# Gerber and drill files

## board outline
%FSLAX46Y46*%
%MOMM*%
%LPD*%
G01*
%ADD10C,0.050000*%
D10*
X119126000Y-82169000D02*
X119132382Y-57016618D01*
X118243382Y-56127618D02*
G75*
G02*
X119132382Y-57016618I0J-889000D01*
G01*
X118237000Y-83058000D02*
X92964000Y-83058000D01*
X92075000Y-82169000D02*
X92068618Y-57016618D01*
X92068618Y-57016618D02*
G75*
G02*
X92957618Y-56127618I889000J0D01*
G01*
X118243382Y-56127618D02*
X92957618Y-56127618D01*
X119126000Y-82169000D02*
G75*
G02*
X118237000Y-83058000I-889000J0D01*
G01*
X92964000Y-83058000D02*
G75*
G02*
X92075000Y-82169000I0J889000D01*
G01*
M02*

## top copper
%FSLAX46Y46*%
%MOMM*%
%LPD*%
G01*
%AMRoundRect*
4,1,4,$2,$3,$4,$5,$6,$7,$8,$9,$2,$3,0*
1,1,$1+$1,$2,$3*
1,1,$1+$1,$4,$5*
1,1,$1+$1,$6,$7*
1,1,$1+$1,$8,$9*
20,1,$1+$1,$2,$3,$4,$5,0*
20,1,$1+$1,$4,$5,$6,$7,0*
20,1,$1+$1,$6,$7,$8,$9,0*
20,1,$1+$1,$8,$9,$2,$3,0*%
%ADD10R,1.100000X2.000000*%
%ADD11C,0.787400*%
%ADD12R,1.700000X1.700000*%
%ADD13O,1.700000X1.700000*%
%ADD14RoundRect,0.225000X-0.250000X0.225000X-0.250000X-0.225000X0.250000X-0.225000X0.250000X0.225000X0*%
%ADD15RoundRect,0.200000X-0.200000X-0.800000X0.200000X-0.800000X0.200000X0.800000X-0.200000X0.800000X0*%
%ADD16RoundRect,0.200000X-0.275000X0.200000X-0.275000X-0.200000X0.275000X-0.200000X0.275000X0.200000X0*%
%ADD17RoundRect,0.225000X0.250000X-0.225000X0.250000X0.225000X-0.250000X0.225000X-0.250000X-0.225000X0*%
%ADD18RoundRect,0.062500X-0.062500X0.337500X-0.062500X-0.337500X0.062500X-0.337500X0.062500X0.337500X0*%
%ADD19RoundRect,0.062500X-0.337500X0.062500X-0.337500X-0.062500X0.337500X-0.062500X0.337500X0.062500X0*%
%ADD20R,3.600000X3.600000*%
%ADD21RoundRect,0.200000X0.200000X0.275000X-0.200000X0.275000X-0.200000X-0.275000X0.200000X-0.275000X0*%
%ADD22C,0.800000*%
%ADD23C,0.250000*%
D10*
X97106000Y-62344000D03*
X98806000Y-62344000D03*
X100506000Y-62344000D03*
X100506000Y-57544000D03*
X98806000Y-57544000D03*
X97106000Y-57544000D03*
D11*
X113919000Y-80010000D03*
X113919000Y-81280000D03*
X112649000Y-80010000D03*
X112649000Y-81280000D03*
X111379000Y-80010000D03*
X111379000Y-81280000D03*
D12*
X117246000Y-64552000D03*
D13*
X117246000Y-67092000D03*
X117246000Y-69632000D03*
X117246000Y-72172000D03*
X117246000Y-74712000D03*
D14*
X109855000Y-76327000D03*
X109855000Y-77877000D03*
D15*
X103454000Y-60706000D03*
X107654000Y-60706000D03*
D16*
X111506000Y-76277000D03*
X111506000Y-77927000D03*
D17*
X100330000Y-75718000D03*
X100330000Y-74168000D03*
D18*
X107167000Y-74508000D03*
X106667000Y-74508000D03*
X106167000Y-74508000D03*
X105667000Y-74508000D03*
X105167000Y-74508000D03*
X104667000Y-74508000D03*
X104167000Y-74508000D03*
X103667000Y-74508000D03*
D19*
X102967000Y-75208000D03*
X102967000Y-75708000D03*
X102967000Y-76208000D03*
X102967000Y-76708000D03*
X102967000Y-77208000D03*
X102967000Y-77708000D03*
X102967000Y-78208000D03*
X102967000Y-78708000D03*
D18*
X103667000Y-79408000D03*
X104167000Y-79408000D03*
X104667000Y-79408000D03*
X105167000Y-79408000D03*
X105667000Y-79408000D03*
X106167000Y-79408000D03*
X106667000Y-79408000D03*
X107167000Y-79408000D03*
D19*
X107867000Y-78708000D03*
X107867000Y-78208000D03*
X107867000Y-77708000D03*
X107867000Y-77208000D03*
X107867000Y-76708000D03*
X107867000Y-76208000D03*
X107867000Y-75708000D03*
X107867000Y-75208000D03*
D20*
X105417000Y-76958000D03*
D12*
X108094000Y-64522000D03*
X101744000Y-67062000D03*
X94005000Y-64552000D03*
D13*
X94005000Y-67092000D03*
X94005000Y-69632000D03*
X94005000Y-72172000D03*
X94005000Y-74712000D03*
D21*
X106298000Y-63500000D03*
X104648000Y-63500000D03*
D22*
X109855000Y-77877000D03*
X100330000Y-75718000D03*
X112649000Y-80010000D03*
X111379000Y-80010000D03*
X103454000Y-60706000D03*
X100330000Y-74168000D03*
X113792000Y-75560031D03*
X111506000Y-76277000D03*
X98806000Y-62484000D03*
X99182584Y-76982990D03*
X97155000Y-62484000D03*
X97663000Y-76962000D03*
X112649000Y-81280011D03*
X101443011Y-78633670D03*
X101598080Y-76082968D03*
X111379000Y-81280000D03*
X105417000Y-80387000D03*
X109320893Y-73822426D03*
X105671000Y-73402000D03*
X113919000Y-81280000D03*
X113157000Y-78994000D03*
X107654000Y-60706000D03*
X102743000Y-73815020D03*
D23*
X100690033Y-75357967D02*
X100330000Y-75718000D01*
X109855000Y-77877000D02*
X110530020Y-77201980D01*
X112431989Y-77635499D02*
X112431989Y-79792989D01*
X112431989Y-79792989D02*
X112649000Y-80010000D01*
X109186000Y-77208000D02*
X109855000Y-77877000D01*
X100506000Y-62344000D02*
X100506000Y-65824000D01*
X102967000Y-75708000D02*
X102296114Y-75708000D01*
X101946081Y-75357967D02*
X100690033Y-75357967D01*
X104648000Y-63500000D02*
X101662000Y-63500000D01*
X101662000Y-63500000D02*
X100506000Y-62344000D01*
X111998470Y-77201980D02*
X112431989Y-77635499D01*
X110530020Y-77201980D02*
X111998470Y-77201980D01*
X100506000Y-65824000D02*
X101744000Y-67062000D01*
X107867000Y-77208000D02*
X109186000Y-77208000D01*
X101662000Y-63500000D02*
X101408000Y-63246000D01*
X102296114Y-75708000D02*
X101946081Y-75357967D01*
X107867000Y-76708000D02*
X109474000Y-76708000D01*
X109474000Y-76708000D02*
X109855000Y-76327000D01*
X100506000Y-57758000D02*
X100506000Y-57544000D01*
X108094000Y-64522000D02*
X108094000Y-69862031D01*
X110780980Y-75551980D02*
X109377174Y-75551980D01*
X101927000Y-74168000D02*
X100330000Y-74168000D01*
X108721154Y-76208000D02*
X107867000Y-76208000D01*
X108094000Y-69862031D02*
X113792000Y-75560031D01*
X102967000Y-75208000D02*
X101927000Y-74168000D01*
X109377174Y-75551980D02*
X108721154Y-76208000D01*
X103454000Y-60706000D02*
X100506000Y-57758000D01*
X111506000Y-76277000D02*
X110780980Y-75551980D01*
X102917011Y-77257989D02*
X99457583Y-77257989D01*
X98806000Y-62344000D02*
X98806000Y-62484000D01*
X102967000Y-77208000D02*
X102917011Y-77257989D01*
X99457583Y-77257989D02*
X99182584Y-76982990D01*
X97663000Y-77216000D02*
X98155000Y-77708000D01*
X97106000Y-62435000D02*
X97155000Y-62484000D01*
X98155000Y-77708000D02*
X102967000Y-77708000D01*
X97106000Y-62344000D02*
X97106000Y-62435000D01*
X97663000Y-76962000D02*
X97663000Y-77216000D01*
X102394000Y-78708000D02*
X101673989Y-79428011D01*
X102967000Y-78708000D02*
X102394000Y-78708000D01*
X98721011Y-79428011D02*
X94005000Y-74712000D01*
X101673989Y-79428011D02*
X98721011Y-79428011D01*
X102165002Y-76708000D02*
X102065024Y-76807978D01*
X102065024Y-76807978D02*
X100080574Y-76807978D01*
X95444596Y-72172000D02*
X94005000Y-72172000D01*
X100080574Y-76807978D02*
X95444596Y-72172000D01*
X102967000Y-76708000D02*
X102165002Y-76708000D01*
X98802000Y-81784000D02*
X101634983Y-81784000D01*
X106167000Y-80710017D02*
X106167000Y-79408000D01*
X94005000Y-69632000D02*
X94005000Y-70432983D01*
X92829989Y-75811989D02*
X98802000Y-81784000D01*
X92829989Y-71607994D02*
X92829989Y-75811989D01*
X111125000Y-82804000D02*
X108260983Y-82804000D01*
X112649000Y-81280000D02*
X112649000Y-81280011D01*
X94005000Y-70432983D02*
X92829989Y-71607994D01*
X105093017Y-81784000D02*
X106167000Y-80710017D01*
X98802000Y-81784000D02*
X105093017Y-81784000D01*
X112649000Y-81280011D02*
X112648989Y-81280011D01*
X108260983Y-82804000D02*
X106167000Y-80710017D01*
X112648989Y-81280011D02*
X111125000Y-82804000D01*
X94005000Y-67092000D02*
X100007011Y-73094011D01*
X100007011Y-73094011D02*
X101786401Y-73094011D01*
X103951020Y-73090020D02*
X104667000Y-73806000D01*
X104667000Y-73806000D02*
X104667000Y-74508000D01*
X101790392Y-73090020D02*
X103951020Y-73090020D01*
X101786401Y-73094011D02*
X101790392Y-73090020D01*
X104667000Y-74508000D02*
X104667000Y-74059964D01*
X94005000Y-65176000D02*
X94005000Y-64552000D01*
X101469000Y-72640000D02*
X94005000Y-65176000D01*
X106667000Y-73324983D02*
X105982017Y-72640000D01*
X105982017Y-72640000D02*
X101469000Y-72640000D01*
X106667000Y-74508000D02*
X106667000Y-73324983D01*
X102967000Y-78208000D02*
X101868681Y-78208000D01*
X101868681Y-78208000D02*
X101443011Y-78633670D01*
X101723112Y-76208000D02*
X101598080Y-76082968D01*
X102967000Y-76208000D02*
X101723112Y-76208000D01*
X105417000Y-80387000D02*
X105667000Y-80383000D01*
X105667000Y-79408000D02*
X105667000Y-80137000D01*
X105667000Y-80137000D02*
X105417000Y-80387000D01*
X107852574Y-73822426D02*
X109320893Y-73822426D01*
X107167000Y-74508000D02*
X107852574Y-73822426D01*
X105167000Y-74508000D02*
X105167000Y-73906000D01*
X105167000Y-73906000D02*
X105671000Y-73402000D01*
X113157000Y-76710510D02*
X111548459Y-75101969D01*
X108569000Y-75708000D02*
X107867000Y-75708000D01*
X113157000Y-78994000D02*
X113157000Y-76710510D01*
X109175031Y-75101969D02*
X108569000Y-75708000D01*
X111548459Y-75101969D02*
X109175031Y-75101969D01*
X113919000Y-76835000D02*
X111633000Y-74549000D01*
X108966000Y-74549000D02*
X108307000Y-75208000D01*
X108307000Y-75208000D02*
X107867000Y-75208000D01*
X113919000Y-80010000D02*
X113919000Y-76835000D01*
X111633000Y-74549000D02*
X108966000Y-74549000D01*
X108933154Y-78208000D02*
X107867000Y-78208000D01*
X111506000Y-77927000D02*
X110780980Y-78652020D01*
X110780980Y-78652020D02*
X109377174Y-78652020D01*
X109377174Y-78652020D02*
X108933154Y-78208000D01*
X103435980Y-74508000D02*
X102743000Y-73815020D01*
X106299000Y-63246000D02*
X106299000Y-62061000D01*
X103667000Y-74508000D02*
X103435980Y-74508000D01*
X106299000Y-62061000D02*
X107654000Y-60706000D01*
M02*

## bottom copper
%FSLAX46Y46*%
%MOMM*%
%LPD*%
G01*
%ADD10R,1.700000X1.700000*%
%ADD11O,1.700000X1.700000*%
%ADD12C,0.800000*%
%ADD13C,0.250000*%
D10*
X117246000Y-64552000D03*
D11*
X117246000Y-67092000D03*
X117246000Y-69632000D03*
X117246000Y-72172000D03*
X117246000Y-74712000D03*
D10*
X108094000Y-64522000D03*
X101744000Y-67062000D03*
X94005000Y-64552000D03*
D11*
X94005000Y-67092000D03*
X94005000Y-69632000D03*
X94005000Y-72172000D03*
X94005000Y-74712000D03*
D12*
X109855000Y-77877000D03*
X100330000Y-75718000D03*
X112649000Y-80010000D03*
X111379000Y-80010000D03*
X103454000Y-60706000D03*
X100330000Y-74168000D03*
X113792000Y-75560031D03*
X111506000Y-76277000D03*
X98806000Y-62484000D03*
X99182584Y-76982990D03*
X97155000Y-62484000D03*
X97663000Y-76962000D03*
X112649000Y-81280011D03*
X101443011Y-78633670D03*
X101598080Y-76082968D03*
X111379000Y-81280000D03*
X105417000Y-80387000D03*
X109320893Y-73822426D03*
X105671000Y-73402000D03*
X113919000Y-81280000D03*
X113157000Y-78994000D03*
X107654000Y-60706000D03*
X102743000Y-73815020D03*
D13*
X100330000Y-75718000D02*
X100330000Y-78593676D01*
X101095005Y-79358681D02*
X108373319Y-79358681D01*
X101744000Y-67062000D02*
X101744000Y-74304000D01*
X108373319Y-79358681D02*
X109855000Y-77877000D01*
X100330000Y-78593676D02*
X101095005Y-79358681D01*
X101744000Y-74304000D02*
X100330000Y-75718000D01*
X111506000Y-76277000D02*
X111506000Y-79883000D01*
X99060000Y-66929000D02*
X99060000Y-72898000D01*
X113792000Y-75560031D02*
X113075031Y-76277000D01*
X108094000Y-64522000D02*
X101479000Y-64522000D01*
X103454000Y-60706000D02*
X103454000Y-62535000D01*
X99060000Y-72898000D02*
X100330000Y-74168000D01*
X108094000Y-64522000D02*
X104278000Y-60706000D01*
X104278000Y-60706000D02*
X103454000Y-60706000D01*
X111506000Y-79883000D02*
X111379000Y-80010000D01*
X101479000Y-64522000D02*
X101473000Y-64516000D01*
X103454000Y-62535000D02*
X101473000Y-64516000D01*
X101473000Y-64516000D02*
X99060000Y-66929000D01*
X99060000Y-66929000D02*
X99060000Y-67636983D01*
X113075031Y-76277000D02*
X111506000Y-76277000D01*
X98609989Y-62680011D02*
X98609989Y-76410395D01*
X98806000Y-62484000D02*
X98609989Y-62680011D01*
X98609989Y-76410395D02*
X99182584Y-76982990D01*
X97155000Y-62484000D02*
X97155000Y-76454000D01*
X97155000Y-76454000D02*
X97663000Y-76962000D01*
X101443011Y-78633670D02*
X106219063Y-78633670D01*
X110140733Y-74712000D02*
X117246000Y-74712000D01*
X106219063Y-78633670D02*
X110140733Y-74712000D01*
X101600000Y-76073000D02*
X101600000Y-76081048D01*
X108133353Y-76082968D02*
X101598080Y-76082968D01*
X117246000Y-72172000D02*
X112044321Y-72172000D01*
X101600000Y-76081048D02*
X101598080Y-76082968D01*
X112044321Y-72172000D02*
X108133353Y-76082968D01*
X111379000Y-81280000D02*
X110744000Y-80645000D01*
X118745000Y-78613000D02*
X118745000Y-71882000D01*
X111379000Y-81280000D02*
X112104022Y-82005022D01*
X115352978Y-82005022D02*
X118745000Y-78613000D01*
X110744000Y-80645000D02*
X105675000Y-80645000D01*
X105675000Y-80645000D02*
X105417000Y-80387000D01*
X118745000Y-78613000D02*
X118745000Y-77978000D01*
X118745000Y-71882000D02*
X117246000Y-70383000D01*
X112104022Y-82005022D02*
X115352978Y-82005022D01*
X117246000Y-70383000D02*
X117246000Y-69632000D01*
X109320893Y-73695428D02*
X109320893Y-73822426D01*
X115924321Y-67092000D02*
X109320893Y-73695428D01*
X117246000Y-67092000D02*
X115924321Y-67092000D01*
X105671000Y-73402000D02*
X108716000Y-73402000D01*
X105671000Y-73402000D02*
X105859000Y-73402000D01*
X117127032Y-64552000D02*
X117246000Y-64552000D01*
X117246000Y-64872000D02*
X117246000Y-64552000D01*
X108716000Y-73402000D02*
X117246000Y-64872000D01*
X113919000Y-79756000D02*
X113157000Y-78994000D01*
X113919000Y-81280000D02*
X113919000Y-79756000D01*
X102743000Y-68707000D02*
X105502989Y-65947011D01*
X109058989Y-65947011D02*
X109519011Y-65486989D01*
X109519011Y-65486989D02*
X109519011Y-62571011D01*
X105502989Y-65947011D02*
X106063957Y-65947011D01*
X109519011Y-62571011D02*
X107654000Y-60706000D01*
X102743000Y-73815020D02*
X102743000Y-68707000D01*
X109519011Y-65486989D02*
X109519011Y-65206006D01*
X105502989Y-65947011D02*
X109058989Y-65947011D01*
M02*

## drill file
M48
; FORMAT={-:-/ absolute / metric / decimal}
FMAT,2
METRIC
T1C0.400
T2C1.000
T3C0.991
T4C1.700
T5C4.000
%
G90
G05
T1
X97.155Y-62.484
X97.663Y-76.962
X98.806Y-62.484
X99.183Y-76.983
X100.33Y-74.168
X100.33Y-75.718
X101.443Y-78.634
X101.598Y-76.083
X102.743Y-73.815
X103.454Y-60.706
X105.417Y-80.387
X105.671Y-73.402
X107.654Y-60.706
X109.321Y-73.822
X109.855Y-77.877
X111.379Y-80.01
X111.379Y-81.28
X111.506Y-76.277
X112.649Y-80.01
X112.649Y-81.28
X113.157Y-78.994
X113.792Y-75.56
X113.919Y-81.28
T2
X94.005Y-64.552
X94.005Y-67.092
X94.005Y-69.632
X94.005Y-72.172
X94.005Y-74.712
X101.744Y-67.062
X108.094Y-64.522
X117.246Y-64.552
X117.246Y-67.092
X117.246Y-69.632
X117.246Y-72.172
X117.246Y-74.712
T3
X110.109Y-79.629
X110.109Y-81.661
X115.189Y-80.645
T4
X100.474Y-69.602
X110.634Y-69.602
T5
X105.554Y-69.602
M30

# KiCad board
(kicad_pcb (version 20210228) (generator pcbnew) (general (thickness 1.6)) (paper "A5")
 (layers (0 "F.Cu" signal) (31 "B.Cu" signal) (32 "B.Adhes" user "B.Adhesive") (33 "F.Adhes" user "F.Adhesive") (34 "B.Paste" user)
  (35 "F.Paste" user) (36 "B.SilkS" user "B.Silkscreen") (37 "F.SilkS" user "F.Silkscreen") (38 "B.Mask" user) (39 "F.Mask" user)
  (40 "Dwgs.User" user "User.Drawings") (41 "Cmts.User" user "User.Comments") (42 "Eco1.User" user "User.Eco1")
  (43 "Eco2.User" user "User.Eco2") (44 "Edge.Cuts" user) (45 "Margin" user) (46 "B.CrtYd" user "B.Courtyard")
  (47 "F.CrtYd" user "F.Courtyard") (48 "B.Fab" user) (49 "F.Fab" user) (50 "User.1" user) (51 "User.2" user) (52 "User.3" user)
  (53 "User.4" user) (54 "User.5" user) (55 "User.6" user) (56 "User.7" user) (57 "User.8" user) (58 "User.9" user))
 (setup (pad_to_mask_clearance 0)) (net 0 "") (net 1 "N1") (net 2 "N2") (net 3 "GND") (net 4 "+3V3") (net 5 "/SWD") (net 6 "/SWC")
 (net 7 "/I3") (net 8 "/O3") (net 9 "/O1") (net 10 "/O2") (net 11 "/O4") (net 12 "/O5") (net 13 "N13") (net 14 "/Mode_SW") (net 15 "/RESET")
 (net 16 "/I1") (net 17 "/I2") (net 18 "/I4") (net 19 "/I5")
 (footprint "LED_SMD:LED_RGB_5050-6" (layer "F.Cu") (at 98.806 59.944 90)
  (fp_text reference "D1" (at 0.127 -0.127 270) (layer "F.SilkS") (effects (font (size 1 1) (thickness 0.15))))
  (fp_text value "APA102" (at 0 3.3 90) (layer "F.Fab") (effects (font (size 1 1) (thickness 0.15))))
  (pad "1" smd rect (at -2.4 -1.7 180) (locked) (size 1.1 2) (layers "F.Cu" "F.Paste" "F.Mask") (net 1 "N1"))
  (pad "2" smd rect (at -2.4 0 180) (locked) (size 1.1 2) (layers "F.Cu" "F.Paste" "F.Mask") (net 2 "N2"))
  (pad "3" smd rect (at -2.4 1.7 180) (locked) (size 1.1 2) (layers "F.Cu" "F.Paste" "F.Mask") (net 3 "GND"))
  (pad "4" smd rect (at 2.4 1.7 180) (locked) (size 1.1 2) (layers "F.Cu" "F.Paste" "F.Mask") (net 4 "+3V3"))
  (pad "5" smd rect (at 2.4 0 180) (locked) (size 1.1 2) (layers "F.Cu" "F.Paste" "F.Mask"))
  (pad "6" smd rect (at 2.4 -1.7 180) (locked) (size 1.1 2) (layers "F.Cu" "F.Paste" "F.Mask")))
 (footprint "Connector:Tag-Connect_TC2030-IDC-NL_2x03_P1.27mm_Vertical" (layer "F.Cu") (at 112.649 80.645 180)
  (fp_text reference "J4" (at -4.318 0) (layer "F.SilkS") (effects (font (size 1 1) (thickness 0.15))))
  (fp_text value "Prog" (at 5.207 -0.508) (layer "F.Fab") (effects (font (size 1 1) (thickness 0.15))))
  (pad "" np_thru_hole circle (at 2.54 1.016 180) (locked) (size 0.9906 0.9906) (drill 0.9906) (layers *.Cu *.Mask))
  (pad "" np_thru_hole circle (at -2.54 0 180) (locked) (size 0.9906 0.9906) (drill 0.9906) (layers *.Cu *.Mask))
  (pad "" np_thru_hole circle (at 2.54 -1.016 180) (locked) (size 0.9906 0.9906) (drill 0.9906) (layers *.Cu *.Mask))
  (pad "1" connect circle (at -1.27 0.635 180) (locked) (size 0.7874 0.7874) (layers "F.Cu" "F.Mask") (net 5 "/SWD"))
  (pad "2" connect circle (at -1.27 -0.635 180) (locked) (size 0.7874 0.7874) (layers "F.Cu" "F.Mask") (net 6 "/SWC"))
  (pad "3" connect circle (at 0 0.635 180) (locked) (size 0.7874 0.7874) (layers "F.Cu" "F.Mask") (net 3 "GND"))
  (pad "4" connect circle (at 0 -0.635 180) (locked) (size 0.7874 0.7874) (layers "F.Cu" "F.Mask") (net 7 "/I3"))
  (pad "5" connect circle (at 1.27 0.635 180) (locked) (size 0.7874 0.7874) (layers "F.Cu" "F.Mask") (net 4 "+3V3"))
  (pad "6" connect circle (at 1.27 -0.635 180) (locked) (size 0.7874 0.7874) (layers "F.Cu" "F.Mask") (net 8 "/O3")))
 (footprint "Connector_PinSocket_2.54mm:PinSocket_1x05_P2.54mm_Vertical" (layer "F.Cu") (at 117.246 64.552)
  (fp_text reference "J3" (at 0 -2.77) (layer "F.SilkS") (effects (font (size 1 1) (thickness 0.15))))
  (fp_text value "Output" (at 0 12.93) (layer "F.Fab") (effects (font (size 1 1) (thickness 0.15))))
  (pad "1" thru_hole rect (at 0 0) (locked) (size 1.7 1.7) (drill 1) (layers *.Cu *.Mask) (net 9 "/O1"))
  (pad "2" thru_hole oval (at 0 2.54) (locked) (size 1.7 1.7) (drill 1) (layers *.Cu *.Mask) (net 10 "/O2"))
  (pad "3" thru_hole oval (at 0 5.08) (locked) (size 1.7 1.7) (drill 1) (layers *.Cu *.Mask) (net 8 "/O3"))
  (pad "4" thru_hole oval (at 0 7.62) (locked) (size 1.7 1.7) (drill 1) (layers *.Cu *.Mask) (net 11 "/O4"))
  (pad "5" thru_hole oval (at 0 10.16) (locked) (size 1.7 1.7) (drill 1) (layers *.Cu *.Mask) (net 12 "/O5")))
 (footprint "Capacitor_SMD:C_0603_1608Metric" (layer "F.Cu") (at 109.855 77.102 -90)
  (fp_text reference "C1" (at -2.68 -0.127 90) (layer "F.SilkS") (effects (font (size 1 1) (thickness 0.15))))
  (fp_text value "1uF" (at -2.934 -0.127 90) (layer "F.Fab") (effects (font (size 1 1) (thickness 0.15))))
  (pad "1" smd roundrect (at -0.775 0 270) (locked) (size 0.9 0.95) (layers "F.Cu" "F.Paste" "F.Mask") (roundrect_rratio 0.25)
   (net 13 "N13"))
  (pad "2" smd roundrect (at 0.775 0 270) (locked) (size 0.9 0.95) (layers "F.Cu" "F.Paste" "F.Mask") (roundrect_rratio 0.25) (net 3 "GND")))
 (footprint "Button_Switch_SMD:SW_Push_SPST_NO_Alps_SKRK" (layer "F.Cu") (at 105.554 60.706)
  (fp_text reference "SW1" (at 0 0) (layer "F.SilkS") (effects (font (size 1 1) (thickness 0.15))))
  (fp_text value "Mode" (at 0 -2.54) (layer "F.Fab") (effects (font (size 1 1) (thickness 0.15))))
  (pad "1" smd roundrect (at -2.1 0) (locked) (size 0.8 2) (layers "F.Cu" "F.Paste" "F.Mask") (roundrect_rratio 0.25) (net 4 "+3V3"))
  (pad "2" smd roundrect (at 2.1 0) (locked) (size 0.8 2) (layers "F.Cu" "F.Paste" "F.Mask") (roundrect_rratio 0.25) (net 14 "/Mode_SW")))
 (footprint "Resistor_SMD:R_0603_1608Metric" (layer "F.Cu") (at 111.506 77.102 -90)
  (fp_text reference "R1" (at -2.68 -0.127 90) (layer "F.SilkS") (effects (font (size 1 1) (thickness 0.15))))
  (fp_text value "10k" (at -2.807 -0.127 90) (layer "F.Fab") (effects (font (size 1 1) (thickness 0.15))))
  (pad "1" smd roundrect (at -0.825 0 270) (locked) (size 0.8 0.95) (layers "F.Cu" "F.Paste" "F.Mask") (roundrect_rratio 0.25)
   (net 4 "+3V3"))
  (pad "2" smd roundrect (at 0.825 0 270) (locked) (size 0.8 0.95) (layers "F.Cu" "F.Paste" "F.Mask") (roundrect_rratio 0.25)
   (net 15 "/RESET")))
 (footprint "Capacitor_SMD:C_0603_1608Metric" (layer "F.Cu") (at 100.33 74.943 90)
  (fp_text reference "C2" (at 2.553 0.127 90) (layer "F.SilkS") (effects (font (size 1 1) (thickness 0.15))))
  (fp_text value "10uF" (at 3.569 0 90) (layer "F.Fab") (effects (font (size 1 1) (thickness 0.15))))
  (pad "1" smd roundrect (at -0.775 0 90) (locked) (size 0.9 0.95) (layers "F.Cu" "F.Paste" "F.Mask") (roundrect_rratio 0.25) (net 3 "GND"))
  (pad "2" smd roundrect (at 0.775 0 90) (locked) (size 0.9 0.95) (layers "F.Cu" "F.Paste" "F.Mask") (roundrect_rratio 0.25) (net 4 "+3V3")))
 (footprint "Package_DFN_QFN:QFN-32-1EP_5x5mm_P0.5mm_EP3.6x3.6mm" (layer "F.Cu") (at 105.417 76.958 -90)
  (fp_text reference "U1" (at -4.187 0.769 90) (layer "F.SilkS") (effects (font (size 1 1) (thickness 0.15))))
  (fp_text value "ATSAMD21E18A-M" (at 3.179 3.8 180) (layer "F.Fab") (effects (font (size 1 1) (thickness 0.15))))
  (pad "" smd roundrect (at -1.2 1.2 270) (locked) (size 0.97 0.97) (layers "F.Paste") (roundrect_rratio 0.25))
  (pad "" smd roundrect (at 0 0 270) (locked) (size 0.97 0.97) (layers "F.Paste") (roundrect_rratio 0.25))
  (pad "" smd roundrect (at 1.2 -1.2 270) (locked) (size 0.97 0.97) (layers "F.Paste") (roundrect_rratio 0.25))
  (pad "" smd roundrect (at -1.2 -1.2 270) (locked) (size 0.97 0.97) (layers "F.Paste") (roundrect_rratio 0.25))
  (pad "" smd roundrect (at 0 1.2 270) (locked) (size 0.97 0.97) (layers "F.Paste") (roundrect_rratio 0.25))
  (pad "" smd roundrect (at 1.2 0 270) (locked) (size 0.97 0.97) (layers "F.Paste") (roundrect_rratio 0.25))
  (pad "" smd roundrect (at -1.2 0 270) (locked) (size 0.97 0.97) (layers "F.Paste") (roundrect_rratio 0.25))
  (pad "" smd roundrect (at 0 -1.2 270) (locked) (size 0.97 0.97) (layers "F.Paste") (roundrect_rratio 0.25))
  (pad "" smd roundrect (at 1.2 1.2 270) (locked) (size 0.97 0.97) (layers "F.Paste") (roundrect_rratio 0.25))
  (pad "1" smd roundrect (at -2.45 -1.75 270) (locked) (size 0.8 0.25) (layers "F.Cu" "F.Paste" "F.Mask") (roundrect_rratio 0.25)
   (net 10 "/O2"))
  (pad "2" smd roundrect (at -2.45 -1.25 270) (locked) (size 0.8 0.25) (layers "F.Cu" "F.Paste" "F.Mask") (roundrect_rratio 0.25)
   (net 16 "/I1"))
  (pad "3" smd roundrect (at -2.45 -0.75 270) (locked) (size 0.8 0.25) (layers "F.Cu" "F.Paste" "F.Mask") (roundrect_rratio 0.25))
  (pad "4" smd roundrect (at -2.45 -0.25 270) (locked) (size 0.8 0.25) (layers "F.Cu" "F.Paste" "F.Mask") (roundrect_rratio 0.25))
  (pad "5" smd roundrect (at -2.45 0.25 270) (locked) (size 0.8 0.25) (layers "F.Cu" "F.Paste" "F.Mask") (roundrect_rratio 0.25)
   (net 9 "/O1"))
  (pad "6" smd roundrect (at -2.45 0.75 270) (locked) (size 0.8 0.25) (layers "F.Cu" "F.Paste" "F.Mask") (roundrect_rratio 0.25)
   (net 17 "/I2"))
  (pad "7" smd roundrect (at -2.45 1.25 270) (locked) (size 0.8 0.25) (layers "F.Cu" "F.Paste" "F.Mask") (roundrect_rratio 0.25))
  (pad "8" smd roundrect (at -2.45 1.75 270) (locked) (size 0.8 0.25) (layers "F.Cu" "F.Paste" "F.Mask") (roundrect_rratio 0.25)
   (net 14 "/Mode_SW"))
  (pad "9" smd roundrect (at -1.75 2.45 270) (locked) (size 0.25 0.8) (layers "F.Cu" "F.Paste" "F.Mask") (roundrect_rratio 0.25)
   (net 4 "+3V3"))
  (pad "10" smd roundrect (at -1.25 2.45 270) (locked) (size 0.25 0.8) (layers "F.Cu" "F.Paste" "F.Mask") (roundrect_rratio 0.25)
   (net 3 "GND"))
  (pad "11" smd roundrect (at -0.75 2.45 270) (locked) (size 0.25 0.8) (layers "F.Cu" "F.Paste" "F.Mask") (roundrect_rratio 0.25)
   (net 11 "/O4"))
  (pad "12" smd roundrect (at -0.25 2.45 270) (locked) (size 0.25 0.8) (layers "F.Cu" "F.Paste" "F.Mask") (roundrect_rratio 0.25)
   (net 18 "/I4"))
  (pad "13" smd roundrect (at 0.25 2.45 270) (locked) (size 0.25 0.8) (layers "F.Cu" "F.Paste" "F.Mask") (roundrect_rratio 0.25)
   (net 2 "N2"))
  (pad "14" smd roundrect (at 0.75 2.45 270) (locked) (size 0.25 0.8) (layers "F.Cu" "F.Paste" "F.Mask") (roundrect_rratio 0.25)
   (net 1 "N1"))
  (pad "15" smd roundrect (at 1.25 2.45 270) (locked) (size 0.25 0.8) (layers "F.Cu" "F.Paste" "F.Mask") (roundrect_rratio 0.25)
   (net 12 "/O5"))
  (pad "16" smd roundrect (at 1.75 2.45 270) (locked) (size 0.25 0.8) (layers "F.Cu" "F.Paste" "F.Mask") (roundrect_rratio 0.25)
   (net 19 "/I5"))
  (pad "17" smd roundrect (at 2.45 1.75 270) (locked) (size 0.8 0.25) (layers "F.Cu" "F.Paste" "F.Mask") (roundrect_rratio 0.25))
  (pad "18" smd roundrect (at 2.45 1.25 270) (locked) (size 0.8 0.25) (layers "F.Cu" "F.Paste" "F.Mask") (roundrect_rratio 0.25))
  (pad "19" smd roundrect (at 2.45 0.75 270) (locked) (size 0.8 0.25) (layers "F.Cu" "F.Paste" "F.Mask") (roundrect_rratio 0.25))
  (pad "20" smd roundrect (at 2.45 0.25 270) (locked) (size 0.8 0.25) (layers "F.Cu" "F.Paste" "F.Mask") (roundrect_rratio 0.25))
  (pad "21" smd roundrect (at 2.45 -0.25 270) (locked) (size 0.8 0.25) (layers "F.Cu" "F.Paste" "F.Mask") (roundrect_rratio 0.25)
   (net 8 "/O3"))
  (pad "22" smd roundrect (at 2.45 -0.75 270) (locked) (size 0.8 0.25) (layers "F.Cu" "F.Paste" "F.Mask") (roundrect_rratio 0.25)
   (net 7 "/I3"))
  (pad "23" smd roundrect (at 2.45 -1.25 270) (locked) (size 0.8 0.25) (layers "F.Cu" "F.Paste" "F.Mask") (roundrect_rratio 0.25))
  (pad "24" smd roundrect (at 2.45 -1.75 270) (locked) (size 0.8 0.25) (layers "F.Cu" "F.Paste" "F.Mask") (roundrect_rratio 0.25))
  (pad "25" smd roundrect (at 1.75 -2.45 270) (locked) (size 0.25 0.8) (layers "F.Cu" "F.Paste" "F.Mask") (roundrect_rratio 0.25))
  (pad "26" smd roundrect (at 1.25 -2.45 270) (locked) (size 0.25 0.8) (layers "F.Cu" "F.Paste" "F.Mask") (roundrect_rratio 0.25)
   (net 15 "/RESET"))
  (pad "27" smd roundrect (at 0.75 -2.45 270) (locked) (size 0.25 0.8) (layers "F.Cu" "F.Paste" "F.Mask") (roundrect_rratio 0.25))
  (pad "28" smd roundrect (at 0.25 -2.45 270) (locked) (size 0.25 0.8) (layers "F.Cu" "F.Paste" "F.Mask") (roundrect_rratio 0.25)
   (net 3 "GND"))
  (pad "29" smd roundrect (at -0.25 -2.45 270) (locked) (size 0.25 0.8) (layers "F.Cu" "F.Paste" "F.Mask") (roundrect_rratio 0.25)
   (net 13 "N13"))
  (pad "30" smd roundrect (at -0.75 -2.45 270) (locked) (size 0.25 0.8) (layers "F.Cu" "F.Paste" "F.Mask") (roundrect_rratio 0.25)
   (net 4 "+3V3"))
  (pad "31" smd roundrect (at -1.25 -2.45 270) (locked) (size 0.25 0.8) (layers "F.Cu" "F.Paste" "F.Mask") (roundrect_rratio 0.25)
   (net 6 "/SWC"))
  (pad "32" smd roundrect (at -1.75 -2.45 270) (locked) (size 0.25 0.8) (layers "F.Cu" "F.Paste" "F.Mask") (roundrect_rratio 0.25)
   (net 5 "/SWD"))
  (pad "33" smd rect (at 0 0 270) (locked) (size 3.6 3.6) (layers "F.Cu" "F.Mask")))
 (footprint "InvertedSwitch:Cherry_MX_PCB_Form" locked (layer "F.Cu") (at 108.094 64.522)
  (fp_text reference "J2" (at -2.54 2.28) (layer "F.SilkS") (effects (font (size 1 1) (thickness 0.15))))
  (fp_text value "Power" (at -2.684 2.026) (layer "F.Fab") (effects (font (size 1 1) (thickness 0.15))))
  (pad "" np_thru_hole circle (at -7.62 5.08) (locked) (size 1.7 1.7) (drill 1.7) (layers *.Cu *.Mask))
  (pad "" np_thru_hole circle (at 2.54 5.08) (locked) (size 1.7 1.7) (drill 1.7) (layers *.Cu *.Mask))
  (pad "" np_thru_hole circle (at -2.54 5.08) (locked) (size 4 4) (drill 4) (layers *.Cu *.Mask))
  (pad "1" thru_hole rect (at 0 0) (locked) (size 1.7 1.7) (drill 1) (layers *.Cu *.Mask) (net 4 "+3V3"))
  (pad "2" thru_hole rect (at -6.35 2.54) (locked) (size 1.7 1.7) (drill 1) (layers *.Cu *.Mask) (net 3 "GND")))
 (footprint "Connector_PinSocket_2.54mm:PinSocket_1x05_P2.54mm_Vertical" (layer "F.Cu") (at 94.005 64.552)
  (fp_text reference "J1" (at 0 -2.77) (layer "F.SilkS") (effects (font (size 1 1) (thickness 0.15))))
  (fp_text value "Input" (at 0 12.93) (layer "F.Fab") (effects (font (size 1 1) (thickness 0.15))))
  (pad "1" thru_hole rect (at 0 0) (locked) (size 1.7 1.7) (drill 1) (layers *.Cu *.Mask) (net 16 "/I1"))
  (pad "2" thru_hole oval (at 0 2.54) (locked) (size 1.7 1.7) (drill 1) (layers *.Cu *.Mask) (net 17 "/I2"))
  (pad "3" thru_hole oval (at 0 5.08) (locked) (size 1.7 1.7) (drill 1) (layers *.Cu *.Mask) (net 7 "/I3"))
  (pad "4" thru_hole oval (at 0 7.62) (locked) (size 1.7 1.7) (drill 1) (layers *.Cu *.Mask) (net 18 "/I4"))
  (pad "5" thru_hole oval (at 0 10.16) (locked) (size 1.7 1.7) (drill 1) (layers *.Cu *.Mask) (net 19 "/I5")))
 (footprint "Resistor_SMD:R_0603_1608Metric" (layer "F.Cu") (at 105.473 63.5 180)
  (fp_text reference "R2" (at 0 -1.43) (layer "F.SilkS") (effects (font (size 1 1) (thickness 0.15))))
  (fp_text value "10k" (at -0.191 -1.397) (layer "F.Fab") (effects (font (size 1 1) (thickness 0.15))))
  (pad "1" smd roundrect (at -0.825 0 180) (locked) (size 0.8 0.95) (layers "F.Cu" "F.Paste" "F.Mask") (roundrect_rratio 0.25)
   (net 14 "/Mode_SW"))
  (pad "2" smd roundrect (at 0.825 0 180) (locked) (size 0.8 0.95) (layers "F.Cu" "F.Paste" "F.Mask") (roundrect_rratio 0.25) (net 3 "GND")))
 (gr_line (start 119.126 82.169) (end 119.132382 57.016618) (layer "Edge.Cuts") (width 0.05))
 (gr_arc (start 118.243382 57.016618) (end 119.132382 57.016618) (angle -90) (layer "Edge.Cuts") (width 0.05))
 (gr_line (start 118.237 83.058) (end 92.964 83.058) (layer "Edge.Cuts") (width 0.05))
 (gr_line (start 92.075 82.169) (end 92.068618 57.016618) (layer "Edge.Cuts") (width 0.05))
 (gr_arc (start 92.957618 57.016618) (end 92.957618 56.127618) (angle -90) (layer "Edge.Cuts") (width 0.05))
 (gr_line (start 118.243382 56.127618) (end 92.957618 56.127618) (layer "Edge.Cuts") (width 0.05))
 (gr_arc (start 118.237 82.169) (end 118.237 83.058) (angle -90) (layer "Edge.Cuts") (width 0.05))
 (gr_arc (start 92.964 82.169) (end 92.075 82.169) (angle -90) (layer "Edge.Cuts") (width 0.05))
 (segment (start 100.690033 75.357967) (end 100.33 75.718) (width 0.25) (layer "F.Cu") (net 3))
 (segment (start 109.855 77.877) (end 110.53002 77.20198) (width 0.25) (layer "F.Cu") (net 3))
 (segment (start 112.431989 77.635499) (end 112.431989 79.792989) (width 0.25) (layer "F.Cu") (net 3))
 (segment (start 112.431989 79.792989) (end 112.649 80.01) (width 0.25) (layer "F.Cu") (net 3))
 (segment (start 109.186 77.208) (end 109.855 77.877) (width 0.25) (layer "F.Cu") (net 3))
 (segment (start 100.506 62.344) (end 100.506 65.824) (width 0.25) (layer "F.Cu") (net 3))
 (segment (start 102.967 75.708) (end 102.296114 75.708) (width 0.25) (layer "F.Cu") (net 3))
 (segment (start 101.946081 75.357967) (end 100.690033 75.357967) (width 0.25) (layer "F.Cu") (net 3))
 (segment (start 104.648 63.5) (end 101.662 63.5) (width 0.25) (layer "F.Cu") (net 3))
 (segment (start 101.662 63.5) (end 100.506 62.344) (width 0.25) (layer "F.Cu") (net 3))
 (segment (start 111.99847 77.20198) (end 112.431989 77.635499) (width 0.25) (layer "F.Cu") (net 3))
 (segment (start 110.53002 77.20198) (end 111.99847 77.20198) (width 0.25) (layer "F.Cu") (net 3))
 (segment (start 100.506 65.824) (end 101.744 67.062) (width 0.25) (layer "F.Cu") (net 3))
 (segment (start 107.867 77.208) (end 109.186 77.208) (width 0.25) (layer "F.Cu") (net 3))
 (segment (start 101.662 63.5) (end 101.408 63.246) (width 0.25) (layer "F.Cu") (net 3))
 (segment (start 102.296114 75.708) (end 101.946081 75.357967) (width 0.25) (layer "F.Cu") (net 3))
 (via (at 109.855 77.877) (size 0.8) (drill 0.4) (layers "F.Cu" "B.Cu") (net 3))
 (via (at 100.33 75.718) (size 0.8) (drill 0.4) (layers "F.Cu" "B.Cu") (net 3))
 (via (at 112.649 80.01) (size 0.8) (drill 0.4) (layers "F.Cu" "B.Cu") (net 3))
 (segment (start 100.33 75.718) (end 100.33 78.593676) (width 0.25) (layer "B.Cu") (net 3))
 (segment (start 101.095005 79.358681) (end 108.373319 79.358681) (width 0.25) (layer "B.Cu") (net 3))
 (segment (start 101.744 67.062) (end 101.744 74.304) (width 0.25) (layer "B.Cu") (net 3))
 (segment (start 108.373319 79.358681) (end 109.855 77.877) (width 0.25) (layer "B.Cu") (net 3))
 (segment (start 100.33 78.593676) (end 101.095005 79.358681) (width 0.25) (layer "B.Cu") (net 3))
 (segment (start 101.744 74.304) (end 100.33 75.718) (width 0.25) (layer "B.Cu") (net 3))
 (segment (start 107.867 76.708) (end 109.474 76.708) (width 0.25) (layer "F.Cu") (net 13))
 (segment (start 109.474 76.708) (end 109.855 76.327) (width 0.25) (layer "F.Cu") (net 13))
 (segment (start 100.506 57.758) (end 100.506 57.544) (width 0.25) (layer "F.Cu") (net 4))
 (segment (start 108.094 64.522) (end 108.094 69.862031) (width 0.25) (layer "F.Cu") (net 4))
 (segment (start 110.78098 75.55198) (end 109.377174 75.55198) (width 0.25) (layer "F.Cu") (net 4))
 (segment (start 101.927 74.168) (end 100.33 74.168) (width 0.25) (layer "F.Cu") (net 4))
 (segment (start 108.721154 76.208) (end 107.867 76.208) (width 0.25) (layer "F.Cu") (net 4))
 (segment (start 108.094 69.862031) (end 113.792 75.560031) (width 0.25) (layer "F.Cu") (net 4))
 (segment (start 102.967 75.208) (end 101.927 74.168) (width 0.25) (layer "F.Cu") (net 4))
 (segment (start 109.377174 75.55198) (end 108.721154 76.208) (width 0.25) (layer "F.Cu") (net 4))
 (segment (start 103.454 60.706) (end 100.506 57.758) (width 0.25) (layer "F.Cu") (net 4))
 (segment (start 111.506 76.277) (end 110.78098 75.55198) (width 0.25) (layer "F.Cu") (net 4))
 (via (at 111.379 80.01) (size 0.8) (drill 0.4) (layers "F.Cu" "B.Cu") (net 4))
 (via (at 103.454 60.706) (size 0.8) (drill 0.4) (layers "F.Cu" "B.Cu") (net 4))
 (via (at 100.33 74.168) (size 0.8) (drill 0.4) (layers "F.Cu" "B.Cu") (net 4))
 (via (at 113.792 75.560031) (size 0.8) (drill 0.4) (layers "F.Cu" "B.Cu") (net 4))
 (via (at 111.506 76.277) (size 0.8) (drill 0.4) (layers "F.Cu" "B.Cu") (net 4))
 (segment (start 111.506 76.277) (end 111.506 79.883) (width 0.25) (layer "B.Cu") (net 4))
 (segment (start 99.06 66.929) (end 99.06 72.898) (width 0.25) (layer "B.Cu") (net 4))
 (segment (start 113.792 75.560031) (end 113.075031 76.277) (width 0.25) (layer "B.Cu") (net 4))
 (segment (start 108.094 64.522) (end 101.479 64.522) (width 0.25) (layer "B.Cu") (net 4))
 (segment (start 103.454 60.706) (end 103.454 62.535) (width 0.25) (layer "B.Cu") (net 4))
 (segment (start 99.06 72.898) (end 100.33 74.168) (width 0.25) (layer "B.Cu") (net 4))
 (segment (start 108.094 64.522) (end 104.278 60.706) (width 0.25) (layer "B.Cu") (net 4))
 (segment (start 104.278 60.706) (end 103.454 60.706) (width 0.25) (layer "B.Cu") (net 4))
 (segment (start 111.506 79.883) (end 111.379 80.01) (width 0.25) (layer "B.Cu") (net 4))
 (segment (start 101.479 64.522) (end 101.473 64.516) (width 0.25) (layer "B.Cu") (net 4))
 (segment (start 103.454 62.535) (end 101.473 64.516) (width 0.25) (layer "B.Cu") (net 4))
 (segment (start 101.473 64.516) (end 99.06 66.929) (width 0.25) (layer "B.Cu") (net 4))
 (segment (start 99.06 66.929) (end 99.06 67.636983) (width 0.25) (layer "B.Cu") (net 4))
 (segment (start 113.075031 76.277) (end 111.506 76.277) (width 0.25) (layer "B.Cu") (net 4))
 (segment (start 102.917011 77.257989) (end 99.457583 77.257989) (width 0.25) (layer "F.Cu") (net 2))
 (segment (start 98.806 62.344) (end 98.806 62.484) (width 0.25) (layer "F.Cu") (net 2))
 (segment (start 102.967 77.208) (end 102.917011 77.257989) (width 0.25) (layer "F.Cu") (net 2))
 (segment (start 99.457583 77.257989) (end 99.182584 76.98299) (width 0.25) (layer "F.Cu") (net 2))
 (via (at 98.806 62.484) (size 0.8) (drill 0.4) (layers "F.Cu" "B.Cu") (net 2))
 (via (at 99.182584 76.98299) (size 0.8) (drill 0.4) (layers "F.Cu" "B.Cu") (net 2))
 (segment (start 98.609989 62.680011) (end 98.609989 76.410395) (width 0.25) (layer "B.Cu") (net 2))
 (segment (start 98.806 62.484) (end 98.609989 62.680011) (width 0.25) (layer "B.Cu") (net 2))
 (segment (start 98.609989 76.410395) (end 99.182584 76.98299) (width 0.25) (layer "B.Cu") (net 2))
 (segment (start 97.663 77.216) (end 98.155 77.708) (width 0.25) (layer "F.Cu") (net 1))
 (segment (start 97.106 62.435) (end 97.155 62.484) (width 0.25) (layer "F.Cu") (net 1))
 (segment (start 98.155 77.708) (end 102.967 77.708) (width 0.25) (layer "F.Cu") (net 1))
 (segment (start 97.106 62.344) (end 97.106 62.435) (width 0.25) (layer "F.Cu") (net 1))
 (segment (start 97.663 76.962) (end 97.663 77.216) (width 0.25) (layer "F.Cu") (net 1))
 (via (at 97.155 62.484) (size 0.8) (drill 0.4) (layers "F.Cu" "B.Cu") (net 1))
 (via (at 97.663 76.962) (size 0.8) (drill 0.4) (layers "F.Cu" "B.Cu") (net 1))
 (segment (start 97.155 62.484) (end 97.155 76.454) (width 0.25) (layer "B.Cu") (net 1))
 (segment (start 97.155 76.454) (end 97.663 76.962) (width 0.25) (layer "B.Cu") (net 1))
 (segment (start 102.394 78.708) (end 101.673989 79.428011) (width 0.25) (layer "F.Cu") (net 19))
 (segment (start 102.967 78.708) (end 102.394 78.708) (width 0.25) (layer "F.Cu") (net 19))
 (segment (start 98.721011 79.428011) (end 94.005 74.712) (width 0.25) (layer "F.Cu") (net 19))
 (segment (start 101.673989 79.428011) (end 98.721011 79.428011) (width 0.25) (layer "F.Cu") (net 19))
 (segment (start 102.165002 76.708) (end 102.065024 76.807978) (width 0.25) (layer "F.Cu") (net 18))
 (segment (start 102.065024 76.807978) (end 100.080574 76.807978) (width 0.25) (layer "F.Cu") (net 18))
 (segment (start 95.444596 72.172) (end 94.005 72.172) (width 0.25) (layer "F.Cu") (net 18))
 (segment (start 100.080574 76.807978) (end 95.444596 72.172) (width 0.25) (layer "F.Cu") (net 18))
 (segment (start 102.967 76.708) (end 102.165002 76.708) (width 0.25) (layer "F.Cu") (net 18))
 (segment (start 98.802 81.784) (end 101.634983 81.784) (width 0.25) (layer "F.Cu") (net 7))
 (segment (start 106.167 80.710017) (end 106.167 79.408) (width 0.25) (layer "F.Cu") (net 7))
 (segment (start 94.005 69.632) (end 94.005 70.432983) (width 0.25) (layer "F.Cu") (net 7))
 (segment (start 92.829989 75.811989) (end 98.802 81.784) (width 0.25) (layer "F.Cu") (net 7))
 (segment (start 92.829989 71.607994) (end 92.829989 75.811989) (width 0.25) (layer "F.Cu") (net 7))
 (segment (start 111.125 82.804) (end 108.260983 82.804) (width 0.25) (layer "F.Cu") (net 7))
 (segment (start 112.649 81.28) (end 112.649 81.280011) (width 0.25) (layer "F.Cu") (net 7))
 (segment (start 94.005 70.432983) (end 92.829989 71.607994) (width 0.25) (layer "F.Cu") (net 7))
 (segment (start 105.093017 81.784) (end 106.167 80.710017) (width 0.25) (layer "F.Cu") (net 7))
 (segment (start 98.802 81.784) (end 105.093017 81.784) (width 0.25) (layer "F.Cu") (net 7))
 (segment (start 112.649 81.280011) (end 112.648989 81.280011) (width 0.25) (layer "F.Cu") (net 7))
 (segment (start 108.260983 82.804) (end 106.167 80.710017) (width 0.25) (layer "F.Cu") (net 7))
 (segment (start 112.648989 81.280011) (end 111.125 82.804) (width 0.25) (layer "F.Cu") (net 7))
 (via (at 112.649 81.280011) (size 0.8) (drill 0.4) (layers "F.Cu" "B.Cu") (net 7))
 (segment (start 94.005 67.092) (end 100.007011 73.094011) (width 0.25) (layer "F.Cu") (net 17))
 (segment (start 100.007011 73.094011) (end 101.786401 73.094011) (width 0.25) (layer "F.Cu") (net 17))
 (segment (start 103.95102 73.09002) (end 104.667 73.806) (width 0.25) (layer "F.Cu") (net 17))
 (segment (start 104.667 73.806) (end 104.667 74.508) (width 0.25) (layer "F.Cu") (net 17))
 (segment (start 101.790392 73.09002) (end 103.95102 73.09002) (width 0.25) (layer "F.Cu") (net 17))
 (segment (start 101.786401 73.094011) (end 101.790392 73.09002) (width 0.25) (layer "F.Cu") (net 17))
 (segment (start 104.667 74.508) (end 104.667 74.059964) (width 0.25) (layer "F.Cu") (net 17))
 (segment (start 94.005 65.176) (end 94.005 64.552) (width 0.25) (layer "F.Cu") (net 16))
 (segment (start 101.469 72.64) (end 94.005 65.176) (width 0.25) (layer "F.Cu") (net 16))
 (segment (start 106.667 73.324983) (end 105.982017 72.64) (width 0.25) (layer "F.Cu") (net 16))
 (segment (start 105.982017 72.64) (end 101.469 72.64) (width 0.25) (layer "F.Cu") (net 16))
 (segment (start 106.667 74.508) (end 106.667 73.324983) (width 0.25) (layer "F.Cu") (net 16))
 (segment (start 102.967 78.208) (end 101.868681 78.208) (width 0.25) (layer "F.Cu") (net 12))
 (segment (start 101.868681 78.208) (end 101.443011 78.63367) (width 0.25) (layer "F.Cu") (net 12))
 (via (at 101.443011 78.63367) (size 0.8) (drill 0.4) (layers "F.Cu" "B.Cu") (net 12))
 (segment (start 101.443011 78.63367) (end 106.219063 78.63367) (width 0.25) (layer "B.Cu") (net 12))
 (segment (start 110.140733 74.712) (end 117.246 74.712) (width 0.25) (layer "B.Cu") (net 12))
 (segment (start 106.219063 78.63367) (end 110.140733 74.712) (width 0.25) (layer "B.Cu") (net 12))
 (segment (start 101.723112 76.208) (end 101.59808 76.082968) (width 0.25) (layer "F.Cu") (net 11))
 (segment (start 102.967 76.208) (end 101.723112 76.208) (width 0.25) (layer "F.Cu") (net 11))
 (via (at 101.59808 76.082968) (size 0.8) (drill 0.4) (layers "F.Cu" "B.Cu") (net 11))
 (segment (start 101.6 76.073) (end 101.6 76.081048) (width 0.25) (layer "B.Cu") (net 11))
 (segment (start 108.133353 76.082968) (end 101.59808 76.082968) (width 0.25) (layer "B.Cu") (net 11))
 (segment (start 117.246 72.172) (end 112.044321 72.172) (width 0.25) (layer "B.Cu") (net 11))
 (segment (start 101.6 76.081048) (end 101.59808 76.082968) (width 0.25) (layer "B.Cu") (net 11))
 (segment (start 112.044321 72.172) (end 108.133353 76.082968) (width 0.25) (layer "B.Cu") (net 11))
 (segment (start 105.417 80.387) (end 105.667 80.383) (width 0.25) (layer "F.Cu") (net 8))
 (segment (start 105.667 79.408) (end 105.667 80.137) (width 0.25) (layer "F.Cu") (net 8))
 (segment (start 105.667 80.137) (end 105.417 80.387) (width 0.25) (layer "F.Cu") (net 8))
 (via (at 111.379 81.28) (size 0.8) (drill 0.4) (layers "F.Cu" "B.Cu") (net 8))
 (via (at 105.417 80.387) (size 0.8) (drill 0.4) (layers "F.Cu" "B.Cu") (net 8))
 (segment (start 111.379 81.28) (end 110.744 80.645) (width 0.25) (layer "B.Cu") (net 8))
 (segment (start 118.745 78.613) (end 118.745 71.882) (width 0.25) (layer "B.Cu") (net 8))
 (segment (start 111.379 81.28) (end 112.104022 82.005022) (width 0.25) (layer "B.Cu") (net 8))
 (segment (start 115.352978 82.005022) (end 118.745 78.613) (width 0.25) (layer "B.Cu") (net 8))
 (segment (start 110.744 80.645) (end 105.675 80.645) (width 0.25) (layer "B.Cu") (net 8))
 (segment (start 105.675 80.645) (end 105.417 80.387) (width 0.25) (layer "B.Cu") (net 8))
 (segment (start 118.745 78.613) (end 118.745 77.978) (width 0.25) (layer "B.Cu") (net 8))
 (segment (start 118.745 71.882) (end 117.246 70.383) (width 0.25) (layer "B.Cu") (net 8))
 (segment (start 112.104022 82.005022) (end 115.352978 82.005022) (width 0.25) (layer "B.Cu") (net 8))
 (segment (start 117.246 70.383) (end 117.246 69.632) (width 0.25) (layer "B.Cu") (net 8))
 (segment (start 107.852574 73.822426) (end 109.320893 73.822426) (width 0.25) (layer "F.Cu") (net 10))
 (segment (start 107.167 74.508) (end 107.852574 73.822426) (width 0.25) (layer "F.Cu") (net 10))
 (via (at 109.320893 73.822426) (size 0.8) (drill 0.4) (layers "F.Cu" "B.Cu") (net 10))
 (segment (start 109.320893 73.695428) (end 109.320893 73.822426) (width 0.25) (layer "B.Cu") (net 10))
 (segment (start 115.924321 67.092) (end 109.320893 73.695428) (width 0.25) (layer "B.Cu") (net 10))
 (segment (start 117.246 67.092) (end 115.924321 67.092) (width 0.25) (layer "B.Cu") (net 10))
 (segment (start 105.167 74.508) (end 105.167 73.906) (width 0.25) (layer "F.Cu") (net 9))
 (segment (start 105.167 73.906) (end 105.671 73.402) (width 0.25) (layer "F.Cu") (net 9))
 (via (at 105.671 73.402) (size 0.8) (drill 0.4) (layers "F.Cu" "B.Cu") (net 9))
 (segment (start 105.671 73.402) (end 108.716 73.402) (width 0.25) (layer "B.Cu") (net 9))
 (segment (start 105.671 73.402) (end 105.859 73.402) (width 0.25) (layer "B.Cu") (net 9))
 (segment (start 117.127032 64.552) (end 117.246 64.552) (width 0.25) (layer "B.Cu") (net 9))
 (segment (start 117.246 64.872) (end 117.246 64.552) (width 0.25) (layer "B.Cu") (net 9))
 (segment (start 108.716 73.402) (end 117.246 64.872) (width 0.25) (layer "B.Cu") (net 9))
 (segment (start 113.157 76.71051) (end 111.548459 75.101969) (width 0.25) (layer "F.Cu") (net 6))
 (segment (start 108.569 75.708) (end 107.867 75.708) (width 0.25) (layer "F.Cu") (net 6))
 (segment (start 113.157 78.994) (end 113.157 76.71051) (width 0.25) (layer "F.Cu") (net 6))
 (segment (start 109.175031 75.101969) (end 108.569 75.708) (width 0.25) (layer "F.Cu") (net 6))
 (segment (start 111.548459 75.101969) (end 109.175031 75.101969) (width 0.25) (layer "F.Cu") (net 6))
 (via (at 113.919 81.28) (size 0.8) (drill 0.4) (layers "F.Cu" "B.Cu") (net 6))
 (via (at 113.157 78.994) (size 0.8) (drill 0.4) (layers "F.Cu" "B.Cu") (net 6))
 (segment (start 113.919 79.756) (end 113.157 78.994) (width 0.25) (layer "B.Cu") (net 6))
 (segment (start 113.919 81.28) (end 113.919 79.756) (width 0.25) (layer "B.Cu") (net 6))
 (segment (start 113.919 76.835) (end 111.633 74.549) (width 0.25) (layer "F.Cu") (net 5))
 (segment (start 108.966 74.549) (end 108.307 75.208) (width 0.25) (layer "F.Cu") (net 5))
 (segment (start 108.307 75.208) (end 107.867 75.208) (width 0.25) (layer "F.Cu") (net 5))
 (segment (start 113.919 80.01) (end 113.919 76.835) (width 0.25) (layer "F.Cu") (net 5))
 (segment (start 111.633 74.549) (end 108.966 74.549) (width 0.25) (layer "F.Cu") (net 5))
 (segment (start 108.933154 78.208) (end 107.867 78.208) (width 0.25) (layer "F.Cu") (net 15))
 (segment (start 111.506 77.927) (end 110.78098 78.65202) (width 0.25) (layer "F.Cu") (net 15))
 (segment (start 110.78098 78.65202) (end 109.377174 78.65202) (width 0.25) (layer "F.Cu") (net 15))
 (segment (start 109.377174 78.65202) (end 108.933154 78.208) (width 0.25) (layer "F.Cu") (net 15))
 (segment (start 103.43598 74.508) (end 102.743 73.81502) (width 0.25) (layer "F.Cu") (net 14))
 (segment (start 106.299 63.246) (end 106.299 62.061) (width 0.25) (layer "F.Cu") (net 14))
 (segment (start 103.667 74.508) (end 103.43598 74.508) (width 0.25) (layer "F.Cu") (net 14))
 (segment (start 106.299 62.061) (end 107.654 60.706) (width 0.25) (layer "F.Cu") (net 14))
 (via (at 107.654 60.706) (size 0.8) (drill 0.4) (layers "F.Cu" "B.Cu") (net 14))
 (via (at 102.743 73.81502) (size 0.8) (drill 0.4) (layers "F.Cu" "B.Cu") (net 14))
 (segment (start 102.743 68.707) (end 105.502989 65.947011) (width 0.25) (layer "B.Cu") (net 14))
 (segment (start 109.058989 65.947011) (end 109.519011 65.486989) (width 0.25) (layer "B.Cu") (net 14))
 (segment (start 109.519011 65.486989) (end 109.519011 62.571011) (width 0.25) (layer "B.Cu") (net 14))
 (segment (start 105.502989 65.947011) (end 106.063957 65.947011) (width 0.25) (layer "B.Cu") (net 14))
 (segment (start 109.519011 62.571011) (end 107.654 60.706) (width 0.25) (layer "B.Cu") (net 14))
 (segment (start 102.743 73.81502) (end 102.743 68.707) (width 0.25) (layer "B.Cu") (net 14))
 (segment (start 109.519011 65.486989) (end 109.519011 65.206006) (width 0.25) (layer "B.Cu") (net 14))
 (segment (start 105.502989 65.947011) (end 109.058989 65.947011) (width 0.25) (layer "B.Cu") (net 14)))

